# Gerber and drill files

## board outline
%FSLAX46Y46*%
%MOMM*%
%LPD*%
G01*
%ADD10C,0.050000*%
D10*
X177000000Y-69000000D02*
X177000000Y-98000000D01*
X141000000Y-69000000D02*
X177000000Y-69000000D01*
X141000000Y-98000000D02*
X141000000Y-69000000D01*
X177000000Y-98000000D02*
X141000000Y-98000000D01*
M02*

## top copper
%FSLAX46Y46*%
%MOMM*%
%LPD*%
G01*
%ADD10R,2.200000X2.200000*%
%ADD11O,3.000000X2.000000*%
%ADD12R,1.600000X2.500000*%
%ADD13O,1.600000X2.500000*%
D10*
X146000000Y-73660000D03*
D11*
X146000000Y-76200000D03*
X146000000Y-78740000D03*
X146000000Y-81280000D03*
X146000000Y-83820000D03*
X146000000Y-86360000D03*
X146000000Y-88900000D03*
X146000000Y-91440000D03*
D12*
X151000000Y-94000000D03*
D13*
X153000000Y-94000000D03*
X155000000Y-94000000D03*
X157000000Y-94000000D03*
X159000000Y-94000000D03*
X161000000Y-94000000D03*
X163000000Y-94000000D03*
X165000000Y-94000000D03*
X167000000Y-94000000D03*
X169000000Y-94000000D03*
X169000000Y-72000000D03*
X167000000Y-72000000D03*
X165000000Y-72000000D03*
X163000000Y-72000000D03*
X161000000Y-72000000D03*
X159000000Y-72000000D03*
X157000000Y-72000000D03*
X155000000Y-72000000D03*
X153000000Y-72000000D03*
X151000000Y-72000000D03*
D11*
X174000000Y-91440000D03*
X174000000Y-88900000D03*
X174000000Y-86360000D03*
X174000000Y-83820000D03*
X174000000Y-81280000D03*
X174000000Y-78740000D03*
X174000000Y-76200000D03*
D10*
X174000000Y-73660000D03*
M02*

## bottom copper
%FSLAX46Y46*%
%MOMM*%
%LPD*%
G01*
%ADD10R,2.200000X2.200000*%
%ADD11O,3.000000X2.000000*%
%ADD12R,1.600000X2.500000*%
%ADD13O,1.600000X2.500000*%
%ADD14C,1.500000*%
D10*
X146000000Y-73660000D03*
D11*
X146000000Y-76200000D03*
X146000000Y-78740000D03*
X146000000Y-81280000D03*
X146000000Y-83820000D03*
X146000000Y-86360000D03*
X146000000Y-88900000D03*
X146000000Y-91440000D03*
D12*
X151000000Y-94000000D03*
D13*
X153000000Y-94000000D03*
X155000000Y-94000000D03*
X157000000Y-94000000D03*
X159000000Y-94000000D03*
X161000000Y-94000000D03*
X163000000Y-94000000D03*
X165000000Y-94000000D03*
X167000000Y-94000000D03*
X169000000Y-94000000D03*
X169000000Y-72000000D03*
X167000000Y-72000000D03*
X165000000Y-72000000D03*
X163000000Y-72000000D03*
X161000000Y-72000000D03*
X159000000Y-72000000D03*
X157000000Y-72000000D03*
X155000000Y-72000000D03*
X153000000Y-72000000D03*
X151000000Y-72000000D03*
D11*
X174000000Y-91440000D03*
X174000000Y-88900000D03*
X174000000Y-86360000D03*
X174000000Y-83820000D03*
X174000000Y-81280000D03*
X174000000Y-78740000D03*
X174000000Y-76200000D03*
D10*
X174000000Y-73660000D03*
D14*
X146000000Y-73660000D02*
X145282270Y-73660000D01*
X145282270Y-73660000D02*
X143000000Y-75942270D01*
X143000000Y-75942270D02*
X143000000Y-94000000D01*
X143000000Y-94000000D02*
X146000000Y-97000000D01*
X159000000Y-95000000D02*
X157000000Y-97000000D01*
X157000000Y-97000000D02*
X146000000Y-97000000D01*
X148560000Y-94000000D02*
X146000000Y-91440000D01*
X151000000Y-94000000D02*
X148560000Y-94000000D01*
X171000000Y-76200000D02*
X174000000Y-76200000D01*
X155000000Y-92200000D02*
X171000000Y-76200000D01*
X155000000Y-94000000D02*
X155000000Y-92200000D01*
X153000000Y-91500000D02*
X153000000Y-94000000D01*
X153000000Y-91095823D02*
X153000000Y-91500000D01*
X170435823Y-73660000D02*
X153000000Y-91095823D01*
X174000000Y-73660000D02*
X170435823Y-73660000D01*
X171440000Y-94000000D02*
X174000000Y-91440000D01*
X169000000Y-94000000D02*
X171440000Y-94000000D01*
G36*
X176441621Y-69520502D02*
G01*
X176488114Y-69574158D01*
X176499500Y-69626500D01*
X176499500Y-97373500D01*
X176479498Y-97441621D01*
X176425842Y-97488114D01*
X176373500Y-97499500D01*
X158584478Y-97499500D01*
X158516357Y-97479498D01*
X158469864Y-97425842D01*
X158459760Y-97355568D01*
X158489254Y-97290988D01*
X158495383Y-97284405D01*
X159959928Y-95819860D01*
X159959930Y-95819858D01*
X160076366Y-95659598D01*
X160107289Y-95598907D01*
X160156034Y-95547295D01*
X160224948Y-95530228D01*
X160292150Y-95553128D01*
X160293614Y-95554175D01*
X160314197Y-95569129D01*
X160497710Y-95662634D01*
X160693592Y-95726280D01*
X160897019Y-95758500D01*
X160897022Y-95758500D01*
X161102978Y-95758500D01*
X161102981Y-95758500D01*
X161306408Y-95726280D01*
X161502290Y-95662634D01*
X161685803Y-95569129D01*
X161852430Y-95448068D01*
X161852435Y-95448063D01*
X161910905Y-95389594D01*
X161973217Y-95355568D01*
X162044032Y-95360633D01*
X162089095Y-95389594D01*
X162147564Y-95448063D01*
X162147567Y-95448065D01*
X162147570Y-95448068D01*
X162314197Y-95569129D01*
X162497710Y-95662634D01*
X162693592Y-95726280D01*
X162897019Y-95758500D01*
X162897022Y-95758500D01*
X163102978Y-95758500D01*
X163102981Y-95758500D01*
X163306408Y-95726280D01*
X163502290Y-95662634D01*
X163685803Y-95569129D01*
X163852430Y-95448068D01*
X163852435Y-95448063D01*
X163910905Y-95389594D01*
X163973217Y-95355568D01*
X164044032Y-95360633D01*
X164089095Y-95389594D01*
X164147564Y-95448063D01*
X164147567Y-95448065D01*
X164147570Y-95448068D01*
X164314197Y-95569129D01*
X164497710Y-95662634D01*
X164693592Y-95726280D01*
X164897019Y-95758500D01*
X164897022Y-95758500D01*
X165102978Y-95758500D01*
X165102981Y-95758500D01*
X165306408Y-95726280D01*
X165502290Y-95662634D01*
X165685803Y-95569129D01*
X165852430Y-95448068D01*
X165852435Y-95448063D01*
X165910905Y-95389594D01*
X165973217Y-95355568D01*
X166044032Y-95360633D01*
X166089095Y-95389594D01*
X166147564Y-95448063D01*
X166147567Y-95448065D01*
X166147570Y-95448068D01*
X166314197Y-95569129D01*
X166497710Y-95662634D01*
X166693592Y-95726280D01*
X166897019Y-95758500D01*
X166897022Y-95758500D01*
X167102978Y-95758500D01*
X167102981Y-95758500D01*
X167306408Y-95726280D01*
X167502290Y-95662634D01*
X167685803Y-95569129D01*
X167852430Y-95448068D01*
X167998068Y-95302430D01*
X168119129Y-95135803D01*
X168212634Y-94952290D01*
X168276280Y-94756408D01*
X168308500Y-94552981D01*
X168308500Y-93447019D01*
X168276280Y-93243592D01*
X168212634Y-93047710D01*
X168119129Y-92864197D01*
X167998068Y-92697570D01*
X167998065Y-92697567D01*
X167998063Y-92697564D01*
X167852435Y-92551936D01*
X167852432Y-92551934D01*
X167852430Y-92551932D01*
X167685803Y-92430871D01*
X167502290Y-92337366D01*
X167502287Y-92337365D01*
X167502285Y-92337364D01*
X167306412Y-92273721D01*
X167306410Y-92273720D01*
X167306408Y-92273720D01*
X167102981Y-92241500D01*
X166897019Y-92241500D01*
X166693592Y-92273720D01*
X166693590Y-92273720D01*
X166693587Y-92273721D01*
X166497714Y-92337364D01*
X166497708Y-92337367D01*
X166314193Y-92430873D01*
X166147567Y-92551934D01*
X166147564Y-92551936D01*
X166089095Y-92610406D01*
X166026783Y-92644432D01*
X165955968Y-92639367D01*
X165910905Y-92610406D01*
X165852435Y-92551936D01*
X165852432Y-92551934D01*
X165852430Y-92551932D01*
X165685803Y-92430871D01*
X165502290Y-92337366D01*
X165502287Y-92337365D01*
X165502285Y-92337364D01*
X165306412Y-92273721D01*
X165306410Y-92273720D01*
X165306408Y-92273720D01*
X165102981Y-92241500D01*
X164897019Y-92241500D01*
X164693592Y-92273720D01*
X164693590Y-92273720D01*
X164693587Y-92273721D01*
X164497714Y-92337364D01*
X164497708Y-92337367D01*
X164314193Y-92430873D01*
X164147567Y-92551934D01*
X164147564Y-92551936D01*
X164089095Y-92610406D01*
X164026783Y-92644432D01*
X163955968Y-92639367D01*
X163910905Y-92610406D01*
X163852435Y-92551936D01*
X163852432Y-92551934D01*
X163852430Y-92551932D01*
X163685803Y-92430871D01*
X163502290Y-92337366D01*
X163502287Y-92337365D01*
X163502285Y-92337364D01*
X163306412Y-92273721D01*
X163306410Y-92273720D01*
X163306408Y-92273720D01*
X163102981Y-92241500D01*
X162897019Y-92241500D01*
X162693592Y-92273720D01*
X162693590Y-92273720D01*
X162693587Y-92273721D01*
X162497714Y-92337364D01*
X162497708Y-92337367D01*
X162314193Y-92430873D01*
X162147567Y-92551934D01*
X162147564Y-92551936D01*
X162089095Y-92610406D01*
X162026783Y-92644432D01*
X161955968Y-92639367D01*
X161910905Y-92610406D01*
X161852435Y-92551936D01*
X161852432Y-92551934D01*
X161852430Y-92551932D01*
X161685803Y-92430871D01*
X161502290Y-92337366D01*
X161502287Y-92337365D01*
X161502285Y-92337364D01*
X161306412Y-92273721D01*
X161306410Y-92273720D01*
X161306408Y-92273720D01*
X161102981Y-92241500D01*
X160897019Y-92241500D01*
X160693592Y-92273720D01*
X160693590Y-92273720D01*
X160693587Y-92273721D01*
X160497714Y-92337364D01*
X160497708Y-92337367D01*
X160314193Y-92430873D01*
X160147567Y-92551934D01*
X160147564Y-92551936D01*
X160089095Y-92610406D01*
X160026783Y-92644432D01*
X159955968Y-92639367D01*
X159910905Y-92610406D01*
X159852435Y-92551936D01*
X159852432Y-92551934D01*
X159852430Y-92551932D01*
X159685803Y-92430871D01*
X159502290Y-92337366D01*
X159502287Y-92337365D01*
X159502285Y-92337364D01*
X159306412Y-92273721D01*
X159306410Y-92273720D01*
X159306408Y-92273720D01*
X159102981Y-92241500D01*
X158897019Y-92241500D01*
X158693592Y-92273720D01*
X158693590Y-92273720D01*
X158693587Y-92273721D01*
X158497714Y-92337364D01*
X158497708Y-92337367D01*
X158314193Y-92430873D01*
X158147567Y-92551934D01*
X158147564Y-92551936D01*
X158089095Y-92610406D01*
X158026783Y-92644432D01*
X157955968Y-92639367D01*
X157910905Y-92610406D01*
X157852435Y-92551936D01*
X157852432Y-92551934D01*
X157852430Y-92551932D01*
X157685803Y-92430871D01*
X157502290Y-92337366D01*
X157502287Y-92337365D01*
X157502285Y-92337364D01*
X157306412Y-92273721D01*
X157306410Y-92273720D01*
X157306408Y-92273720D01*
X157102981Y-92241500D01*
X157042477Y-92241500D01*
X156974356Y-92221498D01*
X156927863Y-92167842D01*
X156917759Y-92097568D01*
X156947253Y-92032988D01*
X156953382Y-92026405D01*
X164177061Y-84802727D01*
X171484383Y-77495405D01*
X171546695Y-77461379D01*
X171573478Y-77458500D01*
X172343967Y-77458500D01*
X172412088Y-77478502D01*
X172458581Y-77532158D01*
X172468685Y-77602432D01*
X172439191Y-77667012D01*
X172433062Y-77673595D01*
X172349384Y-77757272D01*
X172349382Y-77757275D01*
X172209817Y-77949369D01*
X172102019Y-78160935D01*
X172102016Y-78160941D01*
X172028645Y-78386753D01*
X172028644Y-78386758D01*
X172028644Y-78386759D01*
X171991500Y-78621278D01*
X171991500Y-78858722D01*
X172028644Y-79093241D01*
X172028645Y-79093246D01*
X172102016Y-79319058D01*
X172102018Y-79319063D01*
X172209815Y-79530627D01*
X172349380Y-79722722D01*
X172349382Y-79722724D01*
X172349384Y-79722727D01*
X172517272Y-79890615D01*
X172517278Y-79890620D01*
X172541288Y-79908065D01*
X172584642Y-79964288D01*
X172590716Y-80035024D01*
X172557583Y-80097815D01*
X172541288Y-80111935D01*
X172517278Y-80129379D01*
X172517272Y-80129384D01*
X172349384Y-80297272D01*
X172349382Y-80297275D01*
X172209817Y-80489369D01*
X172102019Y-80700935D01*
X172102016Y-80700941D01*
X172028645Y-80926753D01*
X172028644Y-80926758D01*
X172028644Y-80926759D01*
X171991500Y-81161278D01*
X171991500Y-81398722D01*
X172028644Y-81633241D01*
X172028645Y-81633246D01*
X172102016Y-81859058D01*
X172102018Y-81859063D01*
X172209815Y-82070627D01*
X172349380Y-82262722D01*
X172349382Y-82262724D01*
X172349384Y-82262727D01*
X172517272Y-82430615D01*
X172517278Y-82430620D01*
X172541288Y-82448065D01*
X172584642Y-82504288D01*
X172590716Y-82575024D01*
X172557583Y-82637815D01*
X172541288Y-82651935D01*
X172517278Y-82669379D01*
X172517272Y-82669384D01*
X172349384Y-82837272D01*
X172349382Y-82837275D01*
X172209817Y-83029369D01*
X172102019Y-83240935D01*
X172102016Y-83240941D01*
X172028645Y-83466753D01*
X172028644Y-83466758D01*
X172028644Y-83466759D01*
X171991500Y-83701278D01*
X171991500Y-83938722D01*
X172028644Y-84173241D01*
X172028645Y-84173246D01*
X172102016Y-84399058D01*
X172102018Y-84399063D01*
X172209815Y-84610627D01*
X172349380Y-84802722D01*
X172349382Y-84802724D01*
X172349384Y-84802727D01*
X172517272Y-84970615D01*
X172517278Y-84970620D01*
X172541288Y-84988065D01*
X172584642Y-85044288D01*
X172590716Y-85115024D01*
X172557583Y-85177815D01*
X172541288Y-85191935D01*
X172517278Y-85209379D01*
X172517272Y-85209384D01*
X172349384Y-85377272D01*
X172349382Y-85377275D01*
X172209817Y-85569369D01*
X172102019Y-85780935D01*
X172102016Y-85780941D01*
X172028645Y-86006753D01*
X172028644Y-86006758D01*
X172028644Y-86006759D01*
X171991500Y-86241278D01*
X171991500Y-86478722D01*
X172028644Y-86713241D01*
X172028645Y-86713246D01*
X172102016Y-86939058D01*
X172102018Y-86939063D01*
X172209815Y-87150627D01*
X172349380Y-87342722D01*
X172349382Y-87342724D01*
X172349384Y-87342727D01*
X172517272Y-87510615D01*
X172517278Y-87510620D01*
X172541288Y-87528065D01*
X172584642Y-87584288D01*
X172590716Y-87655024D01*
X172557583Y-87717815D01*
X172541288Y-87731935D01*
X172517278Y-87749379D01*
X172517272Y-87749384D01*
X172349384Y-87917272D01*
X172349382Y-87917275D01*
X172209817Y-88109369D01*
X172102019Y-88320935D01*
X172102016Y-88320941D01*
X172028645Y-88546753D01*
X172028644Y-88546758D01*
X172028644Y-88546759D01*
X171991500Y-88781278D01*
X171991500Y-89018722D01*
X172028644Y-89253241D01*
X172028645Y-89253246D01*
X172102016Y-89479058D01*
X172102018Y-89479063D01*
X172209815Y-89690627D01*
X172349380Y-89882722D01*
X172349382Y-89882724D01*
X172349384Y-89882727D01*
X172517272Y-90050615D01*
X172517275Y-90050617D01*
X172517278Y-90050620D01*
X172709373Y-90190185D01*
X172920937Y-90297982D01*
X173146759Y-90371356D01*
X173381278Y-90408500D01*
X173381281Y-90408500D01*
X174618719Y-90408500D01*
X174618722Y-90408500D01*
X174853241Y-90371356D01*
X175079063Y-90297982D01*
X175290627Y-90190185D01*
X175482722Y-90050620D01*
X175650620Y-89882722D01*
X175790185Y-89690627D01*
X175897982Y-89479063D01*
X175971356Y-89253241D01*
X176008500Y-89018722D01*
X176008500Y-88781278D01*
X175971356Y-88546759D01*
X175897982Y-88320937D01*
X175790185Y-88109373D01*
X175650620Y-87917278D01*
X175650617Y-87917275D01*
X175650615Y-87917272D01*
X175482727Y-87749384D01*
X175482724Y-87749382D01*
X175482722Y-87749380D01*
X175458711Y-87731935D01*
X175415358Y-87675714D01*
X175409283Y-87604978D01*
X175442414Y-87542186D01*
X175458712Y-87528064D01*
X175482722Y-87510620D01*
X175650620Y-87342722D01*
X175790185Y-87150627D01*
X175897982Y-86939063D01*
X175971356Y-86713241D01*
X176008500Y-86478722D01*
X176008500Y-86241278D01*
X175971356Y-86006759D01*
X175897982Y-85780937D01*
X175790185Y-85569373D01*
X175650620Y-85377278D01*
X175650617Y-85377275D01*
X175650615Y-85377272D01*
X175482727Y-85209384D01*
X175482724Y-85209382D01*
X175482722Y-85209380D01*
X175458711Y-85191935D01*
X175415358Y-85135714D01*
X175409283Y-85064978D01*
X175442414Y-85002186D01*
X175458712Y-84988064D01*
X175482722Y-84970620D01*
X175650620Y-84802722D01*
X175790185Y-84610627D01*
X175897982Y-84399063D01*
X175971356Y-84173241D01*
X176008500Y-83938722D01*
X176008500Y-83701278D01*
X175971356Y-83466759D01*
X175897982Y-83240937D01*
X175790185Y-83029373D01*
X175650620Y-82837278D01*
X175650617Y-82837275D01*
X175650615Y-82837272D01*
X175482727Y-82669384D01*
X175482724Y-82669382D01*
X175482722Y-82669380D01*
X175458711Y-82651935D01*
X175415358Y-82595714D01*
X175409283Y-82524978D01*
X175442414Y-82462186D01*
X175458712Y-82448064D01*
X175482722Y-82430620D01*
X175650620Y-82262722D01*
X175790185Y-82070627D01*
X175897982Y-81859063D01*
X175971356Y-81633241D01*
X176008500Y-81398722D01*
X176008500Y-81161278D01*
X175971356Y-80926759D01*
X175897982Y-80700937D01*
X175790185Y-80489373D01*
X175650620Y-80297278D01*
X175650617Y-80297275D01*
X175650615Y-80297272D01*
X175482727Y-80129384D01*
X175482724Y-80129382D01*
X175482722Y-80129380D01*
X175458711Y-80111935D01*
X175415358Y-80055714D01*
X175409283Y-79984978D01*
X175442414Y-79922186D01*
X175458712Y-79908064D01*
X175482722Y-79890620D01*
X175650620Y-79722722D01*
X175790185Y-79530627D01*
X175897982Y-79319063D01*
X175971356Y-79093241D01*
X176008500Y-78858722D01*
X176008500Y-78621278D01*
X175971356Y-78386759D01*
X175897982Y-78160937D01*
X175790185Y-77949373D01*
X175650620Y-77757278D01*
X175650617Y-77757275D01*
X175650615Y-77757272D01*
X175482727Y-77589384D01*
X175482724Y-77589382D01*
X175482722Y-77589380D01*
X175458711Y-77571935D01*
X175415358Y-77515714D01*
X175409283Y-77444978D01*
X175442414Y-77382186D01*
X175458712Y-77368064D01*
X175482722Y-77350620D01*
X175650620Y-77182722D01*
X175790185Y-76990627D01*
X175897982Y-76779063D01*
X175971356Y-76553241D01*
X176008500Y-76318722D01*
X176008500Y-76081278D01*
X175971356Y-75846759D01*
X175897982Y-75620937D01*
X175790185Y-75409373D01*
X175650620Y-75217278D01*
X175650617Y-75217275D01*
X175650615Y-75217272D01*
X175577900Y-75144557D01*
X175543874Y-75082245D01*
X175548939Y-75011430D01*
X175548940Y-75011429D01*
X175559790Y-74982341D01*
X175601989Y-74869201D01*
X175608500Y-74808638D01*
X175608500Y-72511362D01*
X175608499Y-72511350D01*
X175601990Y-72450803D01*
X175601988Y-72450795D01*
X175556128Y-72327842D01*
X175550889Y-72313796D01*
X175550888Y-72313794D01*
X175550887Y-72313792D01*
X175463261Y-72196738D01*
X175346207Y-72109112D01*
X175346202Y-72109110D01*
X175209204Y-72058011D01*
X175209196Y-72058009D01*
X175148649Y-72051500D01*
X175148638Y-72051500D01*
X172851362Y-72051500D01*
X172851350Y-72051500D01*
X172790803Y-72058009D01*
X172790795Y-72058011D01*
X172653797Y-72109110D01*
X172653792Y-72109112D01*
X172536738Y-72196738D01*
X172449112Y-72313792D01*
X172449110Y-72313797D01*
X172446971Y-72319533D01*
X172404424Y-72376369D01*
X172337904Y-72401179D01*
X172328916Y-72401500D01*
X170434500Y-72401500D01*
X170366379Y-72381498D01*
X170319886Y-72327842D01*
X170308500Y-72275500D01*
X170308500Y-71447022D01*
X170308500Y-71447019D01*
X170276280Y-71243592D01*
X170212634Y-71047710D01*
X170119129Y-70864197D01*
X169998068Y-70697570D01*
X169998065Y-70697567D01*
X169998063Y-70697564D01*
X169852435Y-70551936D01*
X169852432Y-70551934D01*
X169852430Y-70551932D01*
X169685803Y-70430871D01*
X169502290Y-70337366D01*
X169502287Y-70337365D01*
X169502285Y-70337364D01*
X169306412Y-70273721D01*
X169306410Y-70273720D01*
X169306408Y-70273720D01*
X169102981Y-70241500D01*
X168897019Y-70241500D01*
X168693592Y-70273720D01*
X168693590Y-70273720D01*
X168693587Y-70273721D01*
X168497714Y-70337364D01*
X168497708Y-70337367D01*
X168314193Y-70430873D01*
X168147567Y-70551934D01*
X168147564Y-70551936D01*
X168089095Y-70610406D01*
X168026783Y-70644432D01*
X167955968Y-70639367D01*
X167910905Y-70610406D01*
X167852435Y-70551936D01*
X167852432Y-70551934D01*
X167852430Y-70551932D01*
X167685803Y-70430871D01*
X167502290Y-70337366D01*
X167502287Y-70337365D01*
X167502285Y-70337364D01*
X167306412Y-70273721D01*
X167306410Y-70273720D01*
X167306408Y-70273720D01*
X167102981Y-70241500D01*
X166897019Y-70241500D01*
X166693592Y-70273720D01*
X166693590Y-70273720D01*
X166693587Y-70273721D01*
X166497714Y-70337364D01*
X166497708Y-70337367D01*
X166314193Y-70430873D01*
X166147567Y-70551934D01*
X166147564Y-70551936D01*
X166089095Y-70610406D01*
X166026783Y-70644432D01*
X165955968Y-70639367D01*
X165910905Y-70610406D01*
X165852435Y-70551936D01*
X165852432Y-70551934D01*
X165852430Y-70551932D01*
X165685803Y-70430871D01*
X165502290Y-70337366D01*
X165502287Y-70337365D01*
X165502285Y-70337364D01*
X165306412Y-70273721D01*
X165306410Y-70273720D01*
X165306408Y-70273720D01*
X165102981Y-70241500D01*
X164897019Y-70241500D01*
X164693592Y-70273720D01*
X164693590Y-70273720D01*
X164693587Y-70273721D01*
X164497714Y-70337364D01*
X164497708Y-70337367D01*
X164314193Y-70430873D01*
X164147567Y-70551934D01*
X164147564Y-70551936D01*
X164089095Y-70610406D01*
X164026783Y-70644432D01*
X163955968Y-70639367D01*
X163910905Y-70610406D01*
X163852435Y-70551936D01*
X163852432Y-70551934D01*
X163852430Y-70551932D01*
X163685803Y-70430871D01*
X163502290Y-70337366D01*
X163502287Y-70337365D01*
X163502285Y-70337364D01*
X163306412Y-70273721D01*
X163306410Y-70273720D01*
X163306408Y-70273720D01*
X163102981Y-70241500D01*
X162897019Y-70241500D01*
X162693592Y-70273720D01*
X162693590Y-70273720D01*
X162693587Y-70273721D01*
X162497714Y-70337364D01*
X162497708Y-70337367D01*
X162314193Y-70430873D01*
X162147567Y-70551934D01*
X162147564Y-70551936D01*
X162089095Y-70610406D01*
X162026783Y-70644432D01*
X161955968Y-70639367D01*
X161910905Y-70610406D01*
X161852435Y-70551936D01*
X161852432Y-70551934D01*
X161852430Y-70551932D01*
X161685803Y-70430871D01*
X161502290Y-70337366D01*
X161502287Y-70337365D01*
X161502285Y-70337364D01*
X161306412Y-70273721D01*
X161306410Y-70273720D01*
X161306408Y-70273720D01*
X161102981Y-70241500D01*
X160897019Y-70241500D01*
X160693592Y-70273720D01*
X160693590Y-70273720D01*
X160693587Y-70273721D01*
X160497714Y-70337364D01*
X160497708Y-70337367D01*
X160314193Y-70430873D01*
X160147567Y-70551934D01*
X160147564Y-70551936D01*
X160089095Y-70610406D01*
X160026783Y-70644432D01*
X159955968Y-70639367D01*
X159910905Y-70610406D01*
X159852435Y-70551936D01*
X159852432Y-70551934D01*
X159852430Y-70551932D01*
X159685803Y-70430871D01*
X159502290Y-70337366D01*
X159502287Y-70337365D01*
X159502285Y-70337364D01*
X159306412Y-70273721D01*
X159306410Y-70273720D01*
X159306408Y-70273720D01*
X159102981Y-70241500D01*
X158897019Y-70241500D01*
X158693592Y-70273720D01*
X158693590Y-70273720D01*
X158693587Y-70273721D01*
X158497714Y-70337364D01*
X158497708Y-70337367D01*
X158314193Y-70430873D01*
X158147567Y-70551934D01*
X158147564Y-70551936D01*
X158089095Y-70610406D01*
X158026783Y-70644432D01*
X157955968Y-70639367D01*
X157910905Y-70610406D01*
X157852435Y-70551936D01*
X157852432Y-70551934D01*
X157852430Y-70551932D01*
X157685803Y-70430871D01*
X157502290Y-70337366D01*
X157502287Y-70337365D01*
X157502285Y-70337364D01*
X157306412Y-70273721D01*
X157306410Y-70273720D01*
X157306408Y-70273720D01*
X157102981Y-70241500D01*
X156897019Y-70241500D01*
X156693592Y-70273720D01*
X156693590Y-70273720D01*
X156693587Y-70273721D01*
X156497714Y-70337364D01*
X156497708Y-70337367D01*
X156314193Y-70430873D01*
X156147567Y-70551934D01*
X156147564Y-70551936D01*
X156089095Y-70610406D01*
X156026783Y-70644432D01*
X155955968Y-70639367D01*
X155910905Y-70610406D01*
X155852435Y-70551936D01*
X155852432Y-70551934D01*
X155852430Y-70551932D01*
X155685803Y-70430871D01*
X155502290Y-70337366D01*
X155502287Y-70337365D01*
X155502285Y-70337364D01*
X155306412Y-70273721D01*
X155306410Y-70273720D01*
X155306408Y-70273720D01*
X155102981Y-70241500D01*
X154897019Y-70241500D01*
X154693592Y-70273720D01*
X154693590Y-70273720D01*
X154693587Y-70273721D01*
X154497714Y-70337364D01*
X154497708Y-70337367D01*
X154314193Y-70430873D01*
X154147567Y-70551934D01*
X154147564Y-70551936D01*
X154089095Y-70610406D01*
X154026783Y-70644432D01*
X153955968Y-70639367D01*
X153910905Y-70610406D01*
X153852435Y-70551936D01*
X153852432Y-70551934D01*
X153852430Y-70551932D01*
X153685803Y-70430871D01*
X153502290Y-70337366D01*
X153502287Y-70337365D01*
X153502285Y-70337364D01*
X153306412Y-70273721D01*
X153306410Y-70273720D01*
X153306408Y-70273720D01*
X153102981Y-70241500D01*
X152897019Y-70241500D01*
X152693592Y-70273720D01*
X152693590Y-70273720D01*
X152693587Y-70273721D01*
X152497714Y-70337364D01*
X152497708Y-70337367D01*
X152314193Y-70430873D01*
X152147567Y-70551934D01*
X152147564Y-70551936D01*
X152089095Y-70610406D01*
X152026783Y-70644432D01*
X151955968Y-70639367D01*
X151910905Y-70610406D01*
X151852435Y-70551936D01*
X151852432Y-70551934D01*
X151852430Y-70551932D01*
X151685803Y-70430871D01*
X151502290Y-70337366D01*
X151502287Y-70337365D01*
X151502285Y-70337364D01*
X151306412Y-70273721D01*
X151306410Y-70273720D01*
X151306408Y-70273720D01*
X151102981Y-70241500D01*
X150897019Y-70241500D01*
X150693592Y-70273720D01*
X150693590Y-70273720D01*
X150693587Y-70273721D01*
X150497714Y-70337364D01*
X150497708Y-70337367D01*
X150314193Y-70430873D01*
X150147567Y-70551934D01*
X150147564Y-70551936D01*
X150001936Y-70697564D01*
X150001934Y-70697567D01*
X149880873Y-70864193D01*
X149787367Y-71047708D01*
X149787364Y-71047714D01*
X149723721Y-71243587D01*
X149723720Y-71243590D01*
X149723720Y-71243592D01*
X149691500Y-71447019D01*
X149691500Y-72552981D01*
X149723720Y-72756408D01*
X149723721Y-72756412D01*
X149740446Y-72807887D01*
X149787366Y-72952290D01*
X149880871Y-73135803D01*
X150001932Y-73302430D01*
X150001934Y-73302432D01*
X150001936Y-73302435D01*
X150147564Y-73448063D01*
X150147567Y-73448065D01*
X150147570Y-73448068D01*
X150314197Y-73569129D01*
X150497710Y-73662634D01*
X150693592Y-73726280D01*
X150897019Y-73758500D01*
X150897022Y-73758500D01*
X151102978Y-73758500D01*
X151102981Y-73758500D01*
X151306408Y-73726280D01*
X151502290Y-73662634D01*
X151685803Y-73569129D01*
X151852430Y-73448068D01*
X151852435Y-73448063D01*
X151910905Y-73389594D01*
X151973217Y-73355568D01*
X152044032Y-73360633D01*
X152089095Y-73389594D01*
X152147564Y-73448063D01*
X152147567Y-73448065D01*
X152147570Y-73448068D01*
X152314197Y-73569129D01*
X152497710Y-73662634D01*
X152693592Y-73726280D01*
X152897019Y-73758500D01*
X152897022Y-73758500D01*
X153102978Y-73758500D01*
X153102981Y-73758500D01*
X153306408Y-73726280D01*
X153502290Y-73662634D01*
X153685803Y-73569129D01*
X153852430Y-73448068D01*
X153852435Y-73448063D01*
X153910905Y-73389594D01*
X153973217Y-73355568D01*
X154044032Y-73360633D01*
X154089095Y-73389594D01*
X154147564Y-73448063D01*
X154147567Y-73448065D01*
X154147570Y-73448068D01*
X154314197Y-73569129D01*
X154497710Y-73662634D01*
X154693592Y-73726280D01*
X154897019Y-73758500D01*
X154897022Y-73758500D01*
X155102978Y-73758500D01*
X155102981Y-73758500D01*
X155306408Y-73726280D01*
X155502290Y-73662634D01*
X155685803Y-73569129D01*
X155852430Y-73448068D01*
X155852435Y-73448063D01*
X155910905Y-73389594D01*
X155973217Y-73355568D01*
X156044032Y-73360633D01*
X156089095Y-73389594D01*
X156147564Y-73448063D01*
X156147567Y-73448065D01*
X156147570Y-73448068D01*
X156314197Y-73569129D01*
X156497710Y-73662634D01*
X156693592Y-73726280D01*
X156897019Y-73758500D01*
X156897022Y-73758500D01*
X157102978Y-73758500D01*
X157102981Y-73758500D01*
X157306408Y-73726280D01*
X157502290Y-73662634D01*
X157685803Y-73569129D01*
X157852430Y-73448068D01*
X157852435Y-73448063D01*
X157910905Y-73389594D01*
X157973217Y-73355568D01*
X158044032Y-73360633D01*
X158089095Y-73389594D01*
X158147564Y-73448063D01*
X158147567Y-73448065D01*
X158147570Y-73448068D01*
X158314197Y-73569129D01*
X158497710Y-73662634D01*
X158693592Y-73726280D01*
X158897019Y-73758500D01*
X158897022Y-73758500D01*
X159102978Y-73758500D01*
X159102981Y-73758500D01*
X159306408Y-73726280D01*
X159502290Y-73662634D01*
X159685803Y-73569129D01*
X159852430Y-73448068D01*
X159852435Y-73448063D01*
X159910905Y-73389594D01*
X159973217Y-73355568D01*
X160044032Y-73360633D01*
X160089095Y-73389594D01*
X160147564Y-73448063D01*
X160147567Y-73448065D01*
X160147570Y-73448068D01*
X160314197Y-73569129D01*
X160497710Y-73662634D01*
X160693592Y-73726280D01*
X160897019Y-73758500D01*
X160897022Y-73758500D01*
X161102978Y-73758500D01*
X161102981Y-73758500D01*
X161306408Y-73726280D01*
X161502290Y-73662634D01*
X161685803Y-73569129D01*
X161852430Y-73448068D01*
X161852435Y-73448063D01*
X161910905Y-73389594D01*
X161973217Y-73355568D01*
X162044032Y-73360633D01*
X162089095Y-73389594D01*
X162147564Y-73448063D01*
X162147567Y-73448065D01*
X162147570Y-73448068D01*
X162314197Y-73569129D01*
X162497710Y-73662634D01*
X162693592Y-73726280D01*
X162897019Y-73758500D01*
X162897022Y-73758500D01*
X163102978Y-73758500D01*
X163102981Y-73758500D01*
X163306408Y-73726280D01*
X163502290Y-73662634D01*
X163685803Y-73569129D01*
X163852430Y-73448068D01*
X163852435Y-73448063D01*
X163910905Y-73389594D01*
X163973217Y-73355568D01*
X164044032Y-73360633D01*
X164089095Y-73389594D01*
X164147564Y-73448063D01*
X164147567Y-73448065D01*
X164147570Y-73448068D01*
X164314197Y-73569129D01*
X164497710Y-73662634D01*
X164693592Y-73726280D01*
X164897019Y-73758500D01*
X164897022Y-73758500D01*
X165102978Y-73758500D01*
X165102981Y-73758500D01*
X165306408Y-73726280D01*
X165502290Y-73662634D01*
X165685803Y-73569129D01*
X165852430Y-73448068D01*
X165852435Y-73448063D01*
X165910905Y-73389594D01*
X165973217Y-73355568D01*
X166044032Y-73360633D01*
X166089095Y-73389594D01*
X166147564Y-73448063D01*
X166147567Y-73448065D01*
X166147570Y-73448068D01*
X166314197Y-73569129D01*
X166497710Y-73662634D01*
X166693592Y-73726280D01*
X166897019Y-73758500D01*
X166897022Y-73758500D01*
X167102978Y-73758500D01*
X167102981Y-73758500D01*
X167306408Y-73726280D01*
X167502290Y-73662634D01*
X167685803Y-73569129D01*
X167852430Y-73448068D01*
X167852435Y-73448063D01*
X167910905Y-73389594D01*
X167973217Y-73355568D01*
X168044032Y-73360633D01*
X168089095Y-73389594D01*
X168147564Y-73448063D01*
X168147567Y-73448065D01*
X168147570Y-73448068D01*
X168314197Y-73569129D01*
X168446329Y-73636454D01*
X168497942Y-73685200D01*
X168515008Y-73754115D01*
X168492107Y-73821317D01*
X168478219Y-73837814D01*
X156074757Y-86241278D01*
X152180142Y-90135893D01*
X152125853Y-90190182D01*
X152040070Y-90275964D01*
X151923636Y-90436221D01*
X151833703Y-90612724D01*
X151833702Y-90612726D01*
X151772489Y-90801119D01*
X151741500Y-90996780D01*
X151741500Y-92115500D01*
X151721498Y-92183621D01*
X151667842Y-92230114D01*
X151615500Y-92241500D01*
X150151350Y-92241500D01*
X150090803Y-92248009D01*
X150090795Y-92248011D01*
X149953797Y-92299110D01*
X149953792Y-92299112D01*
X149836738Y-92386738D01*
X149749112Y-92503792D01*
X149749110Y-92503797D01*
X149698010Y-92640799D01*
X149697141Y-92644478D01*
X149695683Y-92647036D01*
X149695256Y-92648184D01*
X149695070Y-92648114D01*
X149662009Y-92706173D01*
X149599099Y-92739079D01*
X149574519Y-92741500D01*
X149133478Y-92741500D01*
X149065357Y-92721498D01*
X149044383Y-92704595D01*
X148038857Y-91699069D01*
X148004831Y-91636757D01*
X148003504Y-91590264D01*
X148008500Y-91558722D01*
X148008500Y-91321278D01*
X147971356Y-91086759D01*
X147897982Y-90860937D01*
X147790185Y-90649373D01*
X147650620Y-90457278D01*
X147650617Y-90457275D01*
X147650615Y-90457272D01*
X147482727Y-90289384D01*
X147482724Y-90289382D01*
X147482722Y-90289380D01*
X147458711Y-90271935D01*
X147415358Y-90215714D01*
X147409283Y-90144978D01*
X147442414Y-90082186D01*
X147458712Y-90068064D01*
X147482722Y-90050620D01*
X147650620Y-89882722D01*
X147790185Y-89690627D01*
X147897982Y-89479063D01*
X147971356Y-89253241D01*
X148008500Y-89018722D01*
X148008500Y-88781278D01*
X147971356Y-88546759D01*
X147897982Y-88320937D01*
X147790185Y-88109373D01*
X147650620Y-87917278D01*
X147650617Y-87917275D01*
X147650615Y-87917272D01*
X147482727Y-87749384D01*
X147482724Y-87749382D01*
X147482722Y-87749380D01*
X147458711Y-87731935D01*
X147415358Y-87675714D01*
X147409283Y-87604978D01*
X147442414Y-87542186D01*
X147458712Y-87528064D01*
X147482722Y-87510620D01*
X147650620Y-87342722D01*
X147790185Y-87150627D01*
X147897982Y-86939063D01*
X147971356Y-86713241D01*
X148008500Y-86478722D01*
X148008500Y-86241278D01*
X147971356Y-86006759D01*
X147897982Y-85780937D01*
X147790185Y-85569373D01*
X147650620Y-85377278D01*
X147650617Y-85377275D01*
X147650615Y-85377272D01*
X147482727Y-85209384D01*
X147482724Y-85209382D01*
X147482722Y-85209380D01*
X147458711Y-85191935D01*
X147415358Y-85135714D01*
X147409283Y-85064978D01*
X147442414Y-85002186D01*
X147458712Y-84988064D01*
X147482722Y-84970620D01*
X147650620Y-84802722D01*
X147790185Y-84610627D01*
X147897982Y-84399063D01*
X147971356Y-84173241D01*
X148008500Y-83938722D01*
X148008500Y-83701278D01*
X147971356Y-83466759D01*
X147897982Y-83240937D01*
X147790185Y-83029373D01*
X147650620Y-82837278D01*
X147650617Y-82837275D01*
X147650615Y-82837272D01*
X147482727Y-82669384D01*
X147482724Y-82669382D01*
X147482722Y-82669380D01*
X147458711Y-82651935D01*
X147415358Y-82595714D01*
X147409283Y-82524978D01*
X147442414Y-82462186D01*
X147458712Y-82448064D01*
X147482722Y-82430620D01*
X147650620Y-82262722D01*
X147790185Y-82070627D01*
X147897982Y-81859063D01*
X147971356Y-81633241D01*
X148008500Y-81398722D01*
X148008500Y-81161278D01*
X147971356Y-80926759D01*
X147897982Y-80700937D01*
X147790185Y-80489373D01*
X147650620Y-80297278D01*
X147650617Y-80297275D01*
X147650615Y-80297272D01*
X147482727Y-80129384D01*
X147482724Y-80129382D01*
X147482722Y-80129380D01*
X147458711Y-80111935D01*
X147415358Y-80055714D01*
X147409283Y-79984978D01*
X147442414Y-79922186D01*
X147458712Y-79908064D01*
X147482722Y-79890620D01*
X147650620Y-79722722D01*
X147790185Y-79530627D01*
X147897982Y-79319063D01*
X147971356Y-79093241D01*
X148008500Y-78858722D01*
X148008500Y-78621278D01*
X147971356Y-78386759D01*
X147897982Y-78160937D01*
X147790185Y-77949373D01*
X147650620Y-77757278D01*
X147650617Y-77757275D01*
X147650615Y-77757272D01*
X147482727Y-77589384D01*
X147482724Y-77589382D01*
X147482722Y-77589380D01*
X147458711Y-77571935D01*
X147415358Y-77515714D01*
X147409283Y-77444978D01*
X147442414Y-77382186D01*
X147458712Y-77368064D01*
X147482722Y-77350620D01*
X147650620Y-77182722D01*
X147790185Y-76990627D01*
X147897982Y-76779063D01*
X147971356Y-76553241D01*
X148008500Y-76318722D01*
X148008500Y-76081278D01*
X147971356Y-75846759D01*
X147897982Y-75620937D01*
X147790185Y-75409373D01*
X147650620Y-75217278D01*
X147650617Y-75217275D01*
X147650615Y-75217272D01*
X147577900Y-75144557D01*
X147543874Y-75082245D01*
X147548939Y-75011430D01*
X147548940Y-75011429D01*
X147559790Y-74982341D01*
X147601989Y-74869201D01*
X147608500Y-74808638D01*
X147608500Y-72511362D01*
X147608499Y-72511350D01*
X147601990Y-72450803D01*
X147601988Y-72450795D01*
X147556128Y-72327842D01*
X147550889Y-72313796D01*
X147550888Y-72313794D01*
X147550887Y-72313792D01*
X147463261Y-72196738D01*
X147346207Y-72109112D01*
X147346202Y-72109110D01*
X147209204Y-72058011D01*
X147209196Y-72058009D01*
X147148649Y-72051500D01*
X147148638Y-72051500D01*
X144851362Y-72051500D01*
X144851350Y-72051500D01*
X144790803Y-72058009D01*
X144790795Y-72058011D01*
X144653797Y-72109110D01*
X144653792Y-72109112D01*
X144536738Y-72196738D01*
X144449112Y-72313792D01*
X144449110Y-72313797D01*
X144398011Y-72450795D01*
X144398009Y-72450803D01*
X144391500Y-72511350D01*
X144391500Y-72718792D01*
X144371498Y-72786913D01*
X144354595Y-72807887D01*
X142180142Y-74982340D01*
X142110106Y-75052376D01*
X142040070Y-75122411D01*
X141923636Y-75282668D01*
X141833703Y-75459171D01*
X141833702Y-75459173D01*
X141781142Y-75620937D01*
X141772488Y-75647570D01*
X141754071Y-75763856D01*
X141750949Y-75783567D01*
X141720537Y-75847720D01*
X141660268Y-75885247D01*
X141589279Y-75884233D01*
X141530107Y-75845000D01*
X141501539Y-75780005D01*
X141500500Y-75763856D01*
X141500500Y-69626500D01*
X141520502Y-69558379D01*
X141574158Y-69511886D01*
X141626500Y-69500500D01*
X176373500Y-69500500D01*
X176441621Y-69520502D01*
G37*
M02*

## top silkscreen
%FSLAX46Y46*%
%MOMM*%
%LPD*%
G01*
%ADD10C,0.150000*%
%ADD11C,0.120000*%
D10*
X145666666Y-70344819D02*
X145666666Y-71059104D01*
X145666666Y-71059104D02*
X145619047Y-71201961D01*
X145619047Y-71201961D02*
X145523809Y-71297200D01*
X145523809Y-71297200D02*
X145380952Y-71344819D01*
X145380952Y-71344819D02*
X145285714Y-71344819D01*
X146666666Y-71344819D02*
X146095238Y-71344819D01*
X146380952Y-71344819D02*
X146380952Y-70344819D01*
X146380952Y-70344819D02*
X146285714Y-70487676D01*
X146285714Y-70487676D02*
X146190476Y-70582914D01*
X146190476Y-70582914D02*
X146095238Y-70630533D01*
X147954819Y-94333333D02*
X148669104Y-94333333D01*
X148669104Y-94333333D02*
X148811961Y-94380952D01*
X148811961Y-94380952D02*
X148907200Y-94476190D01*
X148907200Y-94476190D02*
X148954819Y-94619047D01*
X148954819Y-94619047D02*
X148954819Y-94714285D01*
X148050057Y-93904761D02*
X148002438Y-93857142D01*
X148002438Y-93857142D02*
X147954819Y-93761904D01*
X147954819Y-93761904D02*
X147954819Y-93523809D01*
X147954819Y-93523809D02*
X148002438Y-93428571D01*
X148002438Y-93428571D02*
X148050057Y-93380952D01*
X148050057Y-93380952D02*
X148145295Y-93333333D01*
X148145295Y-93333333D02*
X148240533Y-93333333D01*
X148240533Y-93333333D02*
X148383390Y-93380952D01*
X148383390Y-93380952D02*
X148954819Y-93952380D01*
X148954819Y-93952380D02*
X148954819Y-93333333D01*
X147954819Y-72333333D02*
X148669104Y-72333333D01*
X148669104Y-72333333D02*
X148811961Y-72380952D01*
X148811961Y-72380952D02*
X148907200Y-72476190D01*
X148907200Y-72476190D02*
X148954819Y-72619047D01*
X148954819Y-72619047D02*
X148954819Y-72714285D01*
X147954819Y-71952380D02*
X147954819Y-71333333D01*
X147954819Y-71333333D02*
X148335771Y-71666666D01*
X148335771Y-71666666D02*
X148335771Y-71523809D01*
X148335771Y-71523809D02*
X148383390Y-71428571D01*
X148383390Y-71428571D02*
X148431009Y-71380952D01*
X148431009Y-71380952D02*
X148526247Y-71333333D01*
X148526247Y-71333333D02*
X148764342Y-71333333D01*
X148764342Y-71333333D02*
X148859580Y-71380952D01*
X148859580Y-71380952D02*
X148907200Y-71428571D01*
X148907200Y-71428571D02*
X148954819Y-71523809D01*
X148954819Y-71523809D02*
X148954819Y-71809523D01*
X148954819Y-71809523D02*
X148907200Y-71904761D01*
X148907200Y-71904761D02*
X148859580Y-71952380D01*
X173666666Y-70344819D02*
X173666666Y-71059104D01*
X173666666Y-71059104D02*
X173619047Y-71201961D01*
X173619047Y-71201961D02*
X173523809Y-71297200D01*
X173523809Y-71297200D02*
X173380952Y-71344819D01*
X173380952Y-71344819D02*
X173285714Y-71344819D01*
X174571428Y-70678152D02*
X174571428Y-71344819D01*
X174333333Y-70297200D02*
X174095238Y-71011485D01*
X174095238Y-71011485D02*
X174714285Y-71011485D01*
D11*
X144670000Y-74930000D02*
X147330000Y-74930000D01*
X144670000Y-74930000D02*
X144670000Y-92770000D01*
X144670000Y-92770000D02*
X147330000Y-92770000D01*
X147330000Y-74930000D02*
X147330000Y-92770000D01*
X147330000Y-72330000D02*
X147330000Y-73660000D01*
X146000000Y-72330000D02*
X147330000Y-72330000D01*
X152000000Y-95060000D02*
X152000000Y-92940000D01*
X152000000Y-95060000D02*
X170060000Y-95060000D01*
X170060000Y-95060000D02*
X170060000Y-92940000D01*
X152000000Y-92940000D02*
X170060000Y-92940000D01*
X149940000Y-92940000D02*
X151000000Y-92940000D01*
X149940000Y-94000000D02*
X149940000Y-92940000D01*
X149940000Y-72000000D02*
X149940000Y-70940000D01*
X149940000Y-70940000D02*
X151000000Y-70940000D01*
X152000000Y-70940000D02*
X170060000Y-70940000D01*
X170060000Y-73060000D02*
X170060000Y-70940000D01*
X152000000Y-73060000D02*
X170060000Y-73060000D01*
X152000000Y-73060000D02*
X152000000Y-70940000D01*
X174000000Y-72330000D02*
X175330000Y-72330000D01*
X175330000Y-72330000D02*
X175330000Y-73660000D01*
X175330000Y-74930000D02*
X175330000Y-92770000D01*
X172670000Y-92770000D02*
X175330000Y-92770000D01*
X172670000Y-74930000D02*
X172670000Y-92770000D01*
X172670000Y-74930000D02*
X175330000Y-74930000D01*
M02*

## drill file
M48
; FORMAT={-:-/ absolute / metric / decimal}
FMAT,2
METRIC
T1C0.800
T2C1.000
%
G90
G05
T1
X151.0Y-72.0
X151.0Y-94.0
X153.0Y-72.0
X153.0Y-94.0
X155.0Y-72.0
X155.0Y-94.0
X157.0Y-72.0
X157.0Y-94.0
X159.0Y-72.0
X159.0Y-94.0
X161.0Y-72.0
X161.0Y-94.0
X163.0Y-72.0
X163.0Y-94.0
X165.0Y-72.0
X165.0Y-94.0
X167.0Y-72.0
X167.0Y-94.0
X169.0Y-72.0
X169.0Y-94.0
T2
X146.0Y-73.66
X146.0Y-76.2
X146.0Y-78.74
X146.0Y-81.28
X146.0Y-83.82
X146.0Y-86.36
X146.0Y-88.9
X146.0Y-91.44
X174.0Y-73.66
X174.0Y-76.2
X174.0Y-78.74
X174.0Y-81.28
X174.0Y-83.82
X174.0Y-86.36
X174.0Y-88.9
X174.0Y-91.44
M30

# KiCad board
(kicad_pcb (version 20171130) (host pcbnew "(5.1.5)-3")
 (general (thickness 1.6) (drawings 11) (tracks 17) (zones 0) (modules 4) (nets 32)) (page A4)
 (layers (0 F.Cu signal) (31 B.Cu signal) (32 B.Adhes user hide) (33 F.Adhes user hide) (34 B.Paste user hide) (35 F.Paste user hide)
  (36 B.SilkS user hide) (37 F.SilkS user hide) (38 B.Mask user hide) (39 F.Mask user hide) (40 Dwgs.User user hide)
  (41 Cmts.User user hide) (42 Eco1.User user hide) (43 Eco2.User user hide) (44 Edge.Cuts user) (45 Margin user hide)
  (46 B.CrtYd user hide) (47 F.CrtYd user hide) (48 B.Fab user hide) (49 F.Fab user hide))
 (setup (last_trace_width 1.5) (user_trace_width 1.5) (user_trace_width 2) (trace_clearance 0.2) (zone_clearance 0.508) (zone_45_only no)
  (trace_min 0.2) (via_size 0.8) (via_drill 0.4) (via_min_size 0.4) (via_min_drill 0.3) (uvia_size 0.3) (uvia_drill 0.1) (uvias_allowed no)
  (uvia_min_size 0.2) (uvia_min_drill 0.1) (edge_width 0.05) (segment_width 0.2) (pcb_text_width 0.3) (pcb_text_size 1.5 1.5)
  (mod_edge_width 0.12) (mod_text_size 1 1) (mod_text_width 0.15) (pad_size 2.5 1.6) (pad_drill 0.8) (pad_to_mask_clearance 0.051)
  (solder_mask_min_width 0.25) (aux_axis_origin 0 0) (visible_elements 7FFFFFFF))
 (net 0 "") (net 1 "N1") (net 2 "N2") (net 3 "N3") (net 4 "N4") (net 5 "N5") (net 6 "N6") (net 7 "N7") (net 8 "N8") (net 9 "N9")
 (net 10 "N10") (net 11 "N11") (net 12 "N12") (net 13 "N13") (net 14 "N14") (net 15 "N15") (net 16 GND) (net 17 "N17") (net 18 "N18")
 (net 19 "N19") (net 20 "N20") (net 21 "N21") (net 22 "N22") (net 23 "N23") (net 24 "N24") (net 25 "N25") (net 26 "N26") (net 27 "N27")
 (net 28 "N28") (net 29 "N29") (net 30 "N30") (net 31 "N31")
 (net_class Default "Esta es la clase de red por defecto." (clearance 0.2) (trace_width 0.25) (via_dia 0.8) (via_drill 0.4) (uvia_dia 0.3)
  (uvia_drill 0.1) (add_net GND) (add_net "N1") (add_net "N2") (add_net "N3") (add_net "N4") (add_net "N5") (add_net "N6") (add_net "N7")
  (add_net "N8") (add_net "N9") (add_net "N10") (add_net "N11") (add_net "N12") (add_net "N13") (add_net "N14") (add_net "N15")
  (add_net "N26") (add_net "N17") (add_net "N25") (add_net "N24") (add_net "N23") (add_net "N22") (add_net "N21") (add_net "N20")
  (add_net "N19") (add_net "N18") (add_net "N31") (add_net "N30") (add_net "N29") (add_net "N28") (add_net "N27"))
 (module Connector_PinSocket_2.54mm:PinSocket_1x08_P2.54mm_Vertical (layer F.Cu) (at 146 73.66)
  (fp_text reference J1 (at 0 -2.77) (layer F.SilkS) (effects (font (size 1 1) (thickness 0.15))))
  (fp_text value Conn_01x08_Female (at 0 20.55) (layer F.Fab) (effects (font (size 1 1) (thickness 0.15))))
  (fp_line (start -1.33 1.27) (end 1.33 1.27) (layer F.SilkS) (width 0.12))
  (fp_line (start -1.33 1.27) (end -1.33 19.11) (layer F.SilkS) (width 0.12))
  (fp_line (start -1.33 19.11) (end 1.33 19.11) (layer F.SilkS) (width 0.12))
  (fp_line (start 1.33 1.27) (end 1.33 19.11) (layer F.SilkS) (width 0.12))
  (fp_line (start 1.33 -1.33) (end 1.33 0) (layer F.SilkS) (width 0.12))
  (fp_line (start 0 -1.33) (end 1.33 -1.33) (layer F.SilkS) (width 0.12))
  (pad 1 thru_hole rect (at 0 0) (size 2.2 2.2) (drill 1) (layers *.Cu *.Mask) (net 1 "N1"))
  (pad 2 thru_hole oval (at 0 2.54) (size 3 2) (drill 1) (layers *.Cu *.Mask) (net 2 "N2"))
  (pad 3 thru_hole oval (at 0 5.08) (size 3 2) (drill 1) (layers *.Cu *.Mask) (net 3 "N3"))
  (pad 4 thru_hole oval (at 0 7.62) (size 3 2) (drill 1) (layers *.Cu *.Mask) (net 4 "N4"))
  (pad 5 thru_hole oval (at 0 10.16) (size 3 2) (drill 1) (layers *.Cu *.Mask) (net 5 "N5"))
  (pad 6 thru_hole oval (at 0 12.7) (size 3 2) (drill 1) (layers *.Cu *.Mask) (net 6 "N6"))
  (pad 7 thru_hole oval (at 0 15.24) (size 3 2) (drill 1) (layers *.Cu *.Mask) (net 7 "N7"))
  (pad 8 thru_hole oval (at 0 17.78) (size 3 2) (drill 1) (layers *.Cu *.Mask) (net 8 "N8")))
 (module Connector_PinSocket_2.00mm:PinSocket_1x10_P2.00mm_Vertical (layer F.Cu) (at 151 94 90)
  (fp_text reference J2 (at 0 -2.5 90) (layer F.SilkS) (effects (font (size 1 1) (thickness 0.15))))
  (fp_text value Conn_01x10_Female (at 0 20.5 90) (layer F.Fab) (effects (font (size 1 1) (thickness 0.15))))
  (fp_line (start -1.06 1) (end 1.06 1) (layer F.SilkS) (width 0.12))
  (fp_line (start -1.06 1) (end -1.06 19.06) (layer F.SilkS) (width 0.12))
  (fp_line (start -1.06 19.06) (end 1.06 19.06) (layer F.SilkS) (width 0.12))
  (fp_line (start 1.06 1) (end 1.06 19.06) (layer F.SilkS) (width 0.12))
  (fp_line (start 1.06 -1.06) (end 1.06 0) (layer F.SilkS) (width 0.12))
  (fp_line (start 0 -1.06) (end 1.06 -1.06) (layer F.SilkS) (width 0.12))
  (pad 1 thru_hole rect (at 0 0 90) (size 2.5 1.6) (drill 0.8) (layers *.Cu *.Mask) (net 8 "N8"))
  (pad 2 thru_hole oval (at 0 2 90) (size 2.5 1.6) (drill 0.8) (layers *.Cu *.Mask) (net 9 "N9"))
  (pad 3 thru_hole oval (at 0 4 90) (size 2.5 1.6) (drill 0.8) (layers *.Cu *.Mask) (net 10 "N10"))
  (pad 4 thru_hole oval (at 0 6 90) (size 2.5 1.6) (drill 0.8) (layers *.Cu *.Mask) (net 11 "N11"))
  (pad 5 thru_hole oval (at 0 8 90) (size 2.5 1.6) (drill 0.8) (layers *.Cu *.Mask) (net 1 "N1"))
  (pad 6 thru_hole oval (at 0 10 90) (size 2.5 1.6) (drill 0.8) (layers *.Cu *.Mask) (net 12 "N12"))
  (pad 7 thru_hole oval (at 0 12 90) (size 2.5 1.6) (drill 0.8) (layers *.Cu *.Mask) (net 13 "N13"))
  (pad 8 thru_hole oval (at 0 14 90) (size 2.5 1.6) (drill 0.8) (layers *.Cu *.Mask) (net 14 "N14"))
  (pad 9 thru_hole oval (at 0 16 90) (size 2.5 1.6) (drill 0.8) (layers *.Cu *.Mask) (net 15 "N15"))
  (pad 10 thru_hole oval (at 0 18 90) (size 2.5 1.6) (drill 0.8) (layers *.Cu *.Mask) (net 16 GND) (zone_connect 2)))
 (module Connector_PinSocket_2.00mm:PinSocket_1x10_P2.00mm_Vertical (layer F.Cu) (at 151 72 90)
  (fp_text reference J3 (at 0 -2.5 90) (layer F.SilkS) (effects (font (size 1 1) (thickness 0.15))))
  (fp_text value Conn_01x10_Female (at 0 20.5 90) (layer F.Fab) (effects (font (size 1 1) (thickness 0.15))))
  (fp_line (start 0 -1.06) (end 1.06 -1.06) (layer F.SilkS) (width 0.12))
  (fp_line (start 1.06 -1.06) (end 1.06 0) (layer F.SilkS) (width 0.12))
  (fp_line (start 1.06 1) (end 1.06 19.06) (layer F.SilkS) (width 0.12))
  (fp_line (start -1.06 19.06) (end 1.06 19.06) (layer F.SilkS) (width 0.12))
  (fp_line (start -1.06 1) (end -1.06 19.06) (layer F.SilkS) (width 0.12))
  (fp_line (start -1.06 1) (end 1.06 1) (layer F.SilkS) (width 0.12))
  (pad 10 thru_hole oval (at 0 18 90) (size 2.5 1.6) (drill 0.8) (layers *.Cu *.Mask) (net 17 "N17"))
  (pad 9 thru_hole oval (at 0 16 90) (size 2.5 1.6) (drill 0.8) (layers *.Cu *.Mask) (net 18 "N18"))
  (pad 8 thru_hole oval (at 0 14 90) (size 2.5 1.6) (drill 0.8) (layers *.Cu *.Mask) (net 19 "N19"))
  (pad 7 thru_hole oval (at 0 12 90) (size 2.5 1.6) (drill 0.8) (layers *.Cu *.Mask) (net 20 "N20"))
  (pad 6 thru_hole oval (at 0 10 90) (size 2.5 1.6) (drill 0.8) (layers *.Cu *.Mask) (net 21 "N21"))
  (pad 5 thru_hole oval (at 0 8 90) (size 2.5 1.6) (drill 0.8) (layers *.Cu *.Mask) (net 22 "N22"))
  (pad 4 thru_hole oval (at 0 6 90) (size 2.5 1.6) (drill 0.8) (layers *.Cu *.Mask) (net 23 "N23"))
  (pad 3 thru_hole oval (at 0 4 90) (size 2.5 1.6) (drill 0.8) (layers *.Cu *.Mask) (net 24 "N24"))
  (pad 2 thru_hole oval (at 0 2 90) (size 2.5 1.6) (drill 0.8) (layers *.Cu *.Mask) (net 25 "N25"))
  (pad 1 thru_hole oval (at 0 0 90) (size 2.5 1.6) (drill 0.8) (layers *.Cu *.Mask) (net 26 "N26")))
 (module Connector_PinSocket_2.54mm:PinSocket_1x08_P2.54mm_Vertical (layer F.Cu) (at 174 73.66)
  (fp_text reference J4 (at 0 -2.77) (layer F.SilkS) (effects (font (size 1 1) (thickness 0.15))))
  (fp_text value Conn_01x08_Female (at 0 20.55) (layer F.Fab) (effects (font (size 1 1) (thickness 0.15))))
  (fp_line (start 0 -1.33) (end 1.33 -1.33) (layer F.SilkS) (width 0.12))
  (fp_line (start 1.33 -1.33) (end 1.33 0) (layer F.SilkS) (width 0.12))
  (fp_line (start 1.33 1.27) (end 1.33 19.11) (layer F.SilkS) (width 0.12))
  (fp_line (start -1.33 19.11) (end 1.33 19.11) (layer F.SilkS) (width 0.12))
  (fp_line (start -1.33 1.27) (end -1.33 19.11) (layer F.SilkS) (width 0.12))
  (fp_line (start -1.33 1.27) (end 1.33 1.27) (layer F.SilkS) (width 0.12))
  (pad 8 thru_hole oval (at 0 17.78) (size 3 2) (drill 1) (layers *.Cu *.Mask) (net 16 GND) (zone_connect 2))
  (pad 7 thru_hole oval (at 0 15.24) (size 3 2) (drill 1) (layers *.Cu *.Mask) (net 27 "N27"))
  (pad 6 thru_hole oval (at 0 12.7) (size 3 2) (drill 1) (layers *.Cu *.Mask) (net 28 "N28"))
  (pad 5 thru_hole oval (at 0 10.16) (size 3 2) (drill 1) (layers *.Cu *.Mask) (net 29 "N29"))
  (pad 4 thru_hole oval (at 0 7.62) (size 3 2) (drill 1) (layers *.Cu *.Mask) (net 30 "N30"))
  (pad 3 thru_hole oval (at 0 5.08) (size 3 2) (drill 1) (layers *.Cu *.Mask) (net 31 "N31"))
  (pad 2 thru_hole oval (at 0 2.54) (size 3 2) (drill 1) (layers *.Cu *.Mask) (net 10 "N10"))
  (pad 1 thru_hole rect (at 0 0) (size 2.2 2.2) (drill 1) (layers *.Cu *.Mask) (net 9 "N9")))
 (gr_line (start 177 69) (end 177 98) (layer Edge.Cuts) (width 0.05))
 (gr_line (start 141 69) (end 177 69) (layer Edge.Cuts) (width 0.05))
 (gr_line (start 141 98) (end 141 69) (layer Edge.Cuts) (width 0.05))
 (gr_line (start 177 98) (end 141 98) (layer Edge.Cuts) (width 0.05))
 (segment (start 146 73.66) (end 145.28227 73.66) (width 1.5) (layer B.Cu) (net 1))
 (segment (start 145.28227 73.66) (end 143 75.94227) (width 1.5) (layer B.Cu) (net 1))
 (segment (start 143 75.94227) (end 143 94) (width 1.5) (layer B.Cu) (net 1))
 (segment (start 143 94) (end 146 97) (width 1.5) (layer B.Cu) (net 1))
 (segment (start 159 95) (end 157 97) (width 1.5) (layer B.Cu) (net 1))
 (segment (start 157 97) (end 146 97) (width 1.5) (layer B.Cu) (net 1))
 (segment (start 148.56 94) (end 146 91.44) (width 1.5) (layer B.Cu) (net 8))
 (segment (start 151 94) (end 148.56 94) (width 1.5) (layer B.Cu) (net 8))
 (segment (start 171 76.2) (end 174 76.2) (width 1.5) (layer B.Cu) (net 10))
 (segment (start 155 92.2) (end 171 76.2) (width 1.5) (layer B.Cu) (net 10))
 (segment (start 155 94) (end 155 92.2) (width 1.5) (layer B.Cu) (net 10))
 (segment (start 153 91.5) (end 153 94) (width 1.5) (layer B.Cu) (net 9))
 (segment (start 153 91.095823) (end 153 91.5) (width 1.5) (layer B.Cu) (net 9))
 (segment (start 170.435823 73.66) (end 153 91.095823) (width 1.5) (layer B.Cu) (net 9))
 (segment (start 174 73.66) (end 170.435823 73.66) (width 1.5) (layer B.Cu) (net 9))
 (segment (start 171.44 94) (end 174 91.44) (width 1.5) (layer B.Cu) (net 16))
 (segment (start 169 94) (end 171.44 94) (width 1.5) (layer B.Cu) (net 16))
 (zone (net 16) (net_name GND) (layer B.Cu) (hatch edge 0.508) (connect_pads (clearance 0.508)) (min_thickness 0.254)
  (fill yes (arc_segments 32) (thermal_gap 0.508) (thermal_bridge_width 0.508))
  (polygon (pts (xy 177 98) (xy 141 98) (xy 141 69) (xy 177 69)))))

